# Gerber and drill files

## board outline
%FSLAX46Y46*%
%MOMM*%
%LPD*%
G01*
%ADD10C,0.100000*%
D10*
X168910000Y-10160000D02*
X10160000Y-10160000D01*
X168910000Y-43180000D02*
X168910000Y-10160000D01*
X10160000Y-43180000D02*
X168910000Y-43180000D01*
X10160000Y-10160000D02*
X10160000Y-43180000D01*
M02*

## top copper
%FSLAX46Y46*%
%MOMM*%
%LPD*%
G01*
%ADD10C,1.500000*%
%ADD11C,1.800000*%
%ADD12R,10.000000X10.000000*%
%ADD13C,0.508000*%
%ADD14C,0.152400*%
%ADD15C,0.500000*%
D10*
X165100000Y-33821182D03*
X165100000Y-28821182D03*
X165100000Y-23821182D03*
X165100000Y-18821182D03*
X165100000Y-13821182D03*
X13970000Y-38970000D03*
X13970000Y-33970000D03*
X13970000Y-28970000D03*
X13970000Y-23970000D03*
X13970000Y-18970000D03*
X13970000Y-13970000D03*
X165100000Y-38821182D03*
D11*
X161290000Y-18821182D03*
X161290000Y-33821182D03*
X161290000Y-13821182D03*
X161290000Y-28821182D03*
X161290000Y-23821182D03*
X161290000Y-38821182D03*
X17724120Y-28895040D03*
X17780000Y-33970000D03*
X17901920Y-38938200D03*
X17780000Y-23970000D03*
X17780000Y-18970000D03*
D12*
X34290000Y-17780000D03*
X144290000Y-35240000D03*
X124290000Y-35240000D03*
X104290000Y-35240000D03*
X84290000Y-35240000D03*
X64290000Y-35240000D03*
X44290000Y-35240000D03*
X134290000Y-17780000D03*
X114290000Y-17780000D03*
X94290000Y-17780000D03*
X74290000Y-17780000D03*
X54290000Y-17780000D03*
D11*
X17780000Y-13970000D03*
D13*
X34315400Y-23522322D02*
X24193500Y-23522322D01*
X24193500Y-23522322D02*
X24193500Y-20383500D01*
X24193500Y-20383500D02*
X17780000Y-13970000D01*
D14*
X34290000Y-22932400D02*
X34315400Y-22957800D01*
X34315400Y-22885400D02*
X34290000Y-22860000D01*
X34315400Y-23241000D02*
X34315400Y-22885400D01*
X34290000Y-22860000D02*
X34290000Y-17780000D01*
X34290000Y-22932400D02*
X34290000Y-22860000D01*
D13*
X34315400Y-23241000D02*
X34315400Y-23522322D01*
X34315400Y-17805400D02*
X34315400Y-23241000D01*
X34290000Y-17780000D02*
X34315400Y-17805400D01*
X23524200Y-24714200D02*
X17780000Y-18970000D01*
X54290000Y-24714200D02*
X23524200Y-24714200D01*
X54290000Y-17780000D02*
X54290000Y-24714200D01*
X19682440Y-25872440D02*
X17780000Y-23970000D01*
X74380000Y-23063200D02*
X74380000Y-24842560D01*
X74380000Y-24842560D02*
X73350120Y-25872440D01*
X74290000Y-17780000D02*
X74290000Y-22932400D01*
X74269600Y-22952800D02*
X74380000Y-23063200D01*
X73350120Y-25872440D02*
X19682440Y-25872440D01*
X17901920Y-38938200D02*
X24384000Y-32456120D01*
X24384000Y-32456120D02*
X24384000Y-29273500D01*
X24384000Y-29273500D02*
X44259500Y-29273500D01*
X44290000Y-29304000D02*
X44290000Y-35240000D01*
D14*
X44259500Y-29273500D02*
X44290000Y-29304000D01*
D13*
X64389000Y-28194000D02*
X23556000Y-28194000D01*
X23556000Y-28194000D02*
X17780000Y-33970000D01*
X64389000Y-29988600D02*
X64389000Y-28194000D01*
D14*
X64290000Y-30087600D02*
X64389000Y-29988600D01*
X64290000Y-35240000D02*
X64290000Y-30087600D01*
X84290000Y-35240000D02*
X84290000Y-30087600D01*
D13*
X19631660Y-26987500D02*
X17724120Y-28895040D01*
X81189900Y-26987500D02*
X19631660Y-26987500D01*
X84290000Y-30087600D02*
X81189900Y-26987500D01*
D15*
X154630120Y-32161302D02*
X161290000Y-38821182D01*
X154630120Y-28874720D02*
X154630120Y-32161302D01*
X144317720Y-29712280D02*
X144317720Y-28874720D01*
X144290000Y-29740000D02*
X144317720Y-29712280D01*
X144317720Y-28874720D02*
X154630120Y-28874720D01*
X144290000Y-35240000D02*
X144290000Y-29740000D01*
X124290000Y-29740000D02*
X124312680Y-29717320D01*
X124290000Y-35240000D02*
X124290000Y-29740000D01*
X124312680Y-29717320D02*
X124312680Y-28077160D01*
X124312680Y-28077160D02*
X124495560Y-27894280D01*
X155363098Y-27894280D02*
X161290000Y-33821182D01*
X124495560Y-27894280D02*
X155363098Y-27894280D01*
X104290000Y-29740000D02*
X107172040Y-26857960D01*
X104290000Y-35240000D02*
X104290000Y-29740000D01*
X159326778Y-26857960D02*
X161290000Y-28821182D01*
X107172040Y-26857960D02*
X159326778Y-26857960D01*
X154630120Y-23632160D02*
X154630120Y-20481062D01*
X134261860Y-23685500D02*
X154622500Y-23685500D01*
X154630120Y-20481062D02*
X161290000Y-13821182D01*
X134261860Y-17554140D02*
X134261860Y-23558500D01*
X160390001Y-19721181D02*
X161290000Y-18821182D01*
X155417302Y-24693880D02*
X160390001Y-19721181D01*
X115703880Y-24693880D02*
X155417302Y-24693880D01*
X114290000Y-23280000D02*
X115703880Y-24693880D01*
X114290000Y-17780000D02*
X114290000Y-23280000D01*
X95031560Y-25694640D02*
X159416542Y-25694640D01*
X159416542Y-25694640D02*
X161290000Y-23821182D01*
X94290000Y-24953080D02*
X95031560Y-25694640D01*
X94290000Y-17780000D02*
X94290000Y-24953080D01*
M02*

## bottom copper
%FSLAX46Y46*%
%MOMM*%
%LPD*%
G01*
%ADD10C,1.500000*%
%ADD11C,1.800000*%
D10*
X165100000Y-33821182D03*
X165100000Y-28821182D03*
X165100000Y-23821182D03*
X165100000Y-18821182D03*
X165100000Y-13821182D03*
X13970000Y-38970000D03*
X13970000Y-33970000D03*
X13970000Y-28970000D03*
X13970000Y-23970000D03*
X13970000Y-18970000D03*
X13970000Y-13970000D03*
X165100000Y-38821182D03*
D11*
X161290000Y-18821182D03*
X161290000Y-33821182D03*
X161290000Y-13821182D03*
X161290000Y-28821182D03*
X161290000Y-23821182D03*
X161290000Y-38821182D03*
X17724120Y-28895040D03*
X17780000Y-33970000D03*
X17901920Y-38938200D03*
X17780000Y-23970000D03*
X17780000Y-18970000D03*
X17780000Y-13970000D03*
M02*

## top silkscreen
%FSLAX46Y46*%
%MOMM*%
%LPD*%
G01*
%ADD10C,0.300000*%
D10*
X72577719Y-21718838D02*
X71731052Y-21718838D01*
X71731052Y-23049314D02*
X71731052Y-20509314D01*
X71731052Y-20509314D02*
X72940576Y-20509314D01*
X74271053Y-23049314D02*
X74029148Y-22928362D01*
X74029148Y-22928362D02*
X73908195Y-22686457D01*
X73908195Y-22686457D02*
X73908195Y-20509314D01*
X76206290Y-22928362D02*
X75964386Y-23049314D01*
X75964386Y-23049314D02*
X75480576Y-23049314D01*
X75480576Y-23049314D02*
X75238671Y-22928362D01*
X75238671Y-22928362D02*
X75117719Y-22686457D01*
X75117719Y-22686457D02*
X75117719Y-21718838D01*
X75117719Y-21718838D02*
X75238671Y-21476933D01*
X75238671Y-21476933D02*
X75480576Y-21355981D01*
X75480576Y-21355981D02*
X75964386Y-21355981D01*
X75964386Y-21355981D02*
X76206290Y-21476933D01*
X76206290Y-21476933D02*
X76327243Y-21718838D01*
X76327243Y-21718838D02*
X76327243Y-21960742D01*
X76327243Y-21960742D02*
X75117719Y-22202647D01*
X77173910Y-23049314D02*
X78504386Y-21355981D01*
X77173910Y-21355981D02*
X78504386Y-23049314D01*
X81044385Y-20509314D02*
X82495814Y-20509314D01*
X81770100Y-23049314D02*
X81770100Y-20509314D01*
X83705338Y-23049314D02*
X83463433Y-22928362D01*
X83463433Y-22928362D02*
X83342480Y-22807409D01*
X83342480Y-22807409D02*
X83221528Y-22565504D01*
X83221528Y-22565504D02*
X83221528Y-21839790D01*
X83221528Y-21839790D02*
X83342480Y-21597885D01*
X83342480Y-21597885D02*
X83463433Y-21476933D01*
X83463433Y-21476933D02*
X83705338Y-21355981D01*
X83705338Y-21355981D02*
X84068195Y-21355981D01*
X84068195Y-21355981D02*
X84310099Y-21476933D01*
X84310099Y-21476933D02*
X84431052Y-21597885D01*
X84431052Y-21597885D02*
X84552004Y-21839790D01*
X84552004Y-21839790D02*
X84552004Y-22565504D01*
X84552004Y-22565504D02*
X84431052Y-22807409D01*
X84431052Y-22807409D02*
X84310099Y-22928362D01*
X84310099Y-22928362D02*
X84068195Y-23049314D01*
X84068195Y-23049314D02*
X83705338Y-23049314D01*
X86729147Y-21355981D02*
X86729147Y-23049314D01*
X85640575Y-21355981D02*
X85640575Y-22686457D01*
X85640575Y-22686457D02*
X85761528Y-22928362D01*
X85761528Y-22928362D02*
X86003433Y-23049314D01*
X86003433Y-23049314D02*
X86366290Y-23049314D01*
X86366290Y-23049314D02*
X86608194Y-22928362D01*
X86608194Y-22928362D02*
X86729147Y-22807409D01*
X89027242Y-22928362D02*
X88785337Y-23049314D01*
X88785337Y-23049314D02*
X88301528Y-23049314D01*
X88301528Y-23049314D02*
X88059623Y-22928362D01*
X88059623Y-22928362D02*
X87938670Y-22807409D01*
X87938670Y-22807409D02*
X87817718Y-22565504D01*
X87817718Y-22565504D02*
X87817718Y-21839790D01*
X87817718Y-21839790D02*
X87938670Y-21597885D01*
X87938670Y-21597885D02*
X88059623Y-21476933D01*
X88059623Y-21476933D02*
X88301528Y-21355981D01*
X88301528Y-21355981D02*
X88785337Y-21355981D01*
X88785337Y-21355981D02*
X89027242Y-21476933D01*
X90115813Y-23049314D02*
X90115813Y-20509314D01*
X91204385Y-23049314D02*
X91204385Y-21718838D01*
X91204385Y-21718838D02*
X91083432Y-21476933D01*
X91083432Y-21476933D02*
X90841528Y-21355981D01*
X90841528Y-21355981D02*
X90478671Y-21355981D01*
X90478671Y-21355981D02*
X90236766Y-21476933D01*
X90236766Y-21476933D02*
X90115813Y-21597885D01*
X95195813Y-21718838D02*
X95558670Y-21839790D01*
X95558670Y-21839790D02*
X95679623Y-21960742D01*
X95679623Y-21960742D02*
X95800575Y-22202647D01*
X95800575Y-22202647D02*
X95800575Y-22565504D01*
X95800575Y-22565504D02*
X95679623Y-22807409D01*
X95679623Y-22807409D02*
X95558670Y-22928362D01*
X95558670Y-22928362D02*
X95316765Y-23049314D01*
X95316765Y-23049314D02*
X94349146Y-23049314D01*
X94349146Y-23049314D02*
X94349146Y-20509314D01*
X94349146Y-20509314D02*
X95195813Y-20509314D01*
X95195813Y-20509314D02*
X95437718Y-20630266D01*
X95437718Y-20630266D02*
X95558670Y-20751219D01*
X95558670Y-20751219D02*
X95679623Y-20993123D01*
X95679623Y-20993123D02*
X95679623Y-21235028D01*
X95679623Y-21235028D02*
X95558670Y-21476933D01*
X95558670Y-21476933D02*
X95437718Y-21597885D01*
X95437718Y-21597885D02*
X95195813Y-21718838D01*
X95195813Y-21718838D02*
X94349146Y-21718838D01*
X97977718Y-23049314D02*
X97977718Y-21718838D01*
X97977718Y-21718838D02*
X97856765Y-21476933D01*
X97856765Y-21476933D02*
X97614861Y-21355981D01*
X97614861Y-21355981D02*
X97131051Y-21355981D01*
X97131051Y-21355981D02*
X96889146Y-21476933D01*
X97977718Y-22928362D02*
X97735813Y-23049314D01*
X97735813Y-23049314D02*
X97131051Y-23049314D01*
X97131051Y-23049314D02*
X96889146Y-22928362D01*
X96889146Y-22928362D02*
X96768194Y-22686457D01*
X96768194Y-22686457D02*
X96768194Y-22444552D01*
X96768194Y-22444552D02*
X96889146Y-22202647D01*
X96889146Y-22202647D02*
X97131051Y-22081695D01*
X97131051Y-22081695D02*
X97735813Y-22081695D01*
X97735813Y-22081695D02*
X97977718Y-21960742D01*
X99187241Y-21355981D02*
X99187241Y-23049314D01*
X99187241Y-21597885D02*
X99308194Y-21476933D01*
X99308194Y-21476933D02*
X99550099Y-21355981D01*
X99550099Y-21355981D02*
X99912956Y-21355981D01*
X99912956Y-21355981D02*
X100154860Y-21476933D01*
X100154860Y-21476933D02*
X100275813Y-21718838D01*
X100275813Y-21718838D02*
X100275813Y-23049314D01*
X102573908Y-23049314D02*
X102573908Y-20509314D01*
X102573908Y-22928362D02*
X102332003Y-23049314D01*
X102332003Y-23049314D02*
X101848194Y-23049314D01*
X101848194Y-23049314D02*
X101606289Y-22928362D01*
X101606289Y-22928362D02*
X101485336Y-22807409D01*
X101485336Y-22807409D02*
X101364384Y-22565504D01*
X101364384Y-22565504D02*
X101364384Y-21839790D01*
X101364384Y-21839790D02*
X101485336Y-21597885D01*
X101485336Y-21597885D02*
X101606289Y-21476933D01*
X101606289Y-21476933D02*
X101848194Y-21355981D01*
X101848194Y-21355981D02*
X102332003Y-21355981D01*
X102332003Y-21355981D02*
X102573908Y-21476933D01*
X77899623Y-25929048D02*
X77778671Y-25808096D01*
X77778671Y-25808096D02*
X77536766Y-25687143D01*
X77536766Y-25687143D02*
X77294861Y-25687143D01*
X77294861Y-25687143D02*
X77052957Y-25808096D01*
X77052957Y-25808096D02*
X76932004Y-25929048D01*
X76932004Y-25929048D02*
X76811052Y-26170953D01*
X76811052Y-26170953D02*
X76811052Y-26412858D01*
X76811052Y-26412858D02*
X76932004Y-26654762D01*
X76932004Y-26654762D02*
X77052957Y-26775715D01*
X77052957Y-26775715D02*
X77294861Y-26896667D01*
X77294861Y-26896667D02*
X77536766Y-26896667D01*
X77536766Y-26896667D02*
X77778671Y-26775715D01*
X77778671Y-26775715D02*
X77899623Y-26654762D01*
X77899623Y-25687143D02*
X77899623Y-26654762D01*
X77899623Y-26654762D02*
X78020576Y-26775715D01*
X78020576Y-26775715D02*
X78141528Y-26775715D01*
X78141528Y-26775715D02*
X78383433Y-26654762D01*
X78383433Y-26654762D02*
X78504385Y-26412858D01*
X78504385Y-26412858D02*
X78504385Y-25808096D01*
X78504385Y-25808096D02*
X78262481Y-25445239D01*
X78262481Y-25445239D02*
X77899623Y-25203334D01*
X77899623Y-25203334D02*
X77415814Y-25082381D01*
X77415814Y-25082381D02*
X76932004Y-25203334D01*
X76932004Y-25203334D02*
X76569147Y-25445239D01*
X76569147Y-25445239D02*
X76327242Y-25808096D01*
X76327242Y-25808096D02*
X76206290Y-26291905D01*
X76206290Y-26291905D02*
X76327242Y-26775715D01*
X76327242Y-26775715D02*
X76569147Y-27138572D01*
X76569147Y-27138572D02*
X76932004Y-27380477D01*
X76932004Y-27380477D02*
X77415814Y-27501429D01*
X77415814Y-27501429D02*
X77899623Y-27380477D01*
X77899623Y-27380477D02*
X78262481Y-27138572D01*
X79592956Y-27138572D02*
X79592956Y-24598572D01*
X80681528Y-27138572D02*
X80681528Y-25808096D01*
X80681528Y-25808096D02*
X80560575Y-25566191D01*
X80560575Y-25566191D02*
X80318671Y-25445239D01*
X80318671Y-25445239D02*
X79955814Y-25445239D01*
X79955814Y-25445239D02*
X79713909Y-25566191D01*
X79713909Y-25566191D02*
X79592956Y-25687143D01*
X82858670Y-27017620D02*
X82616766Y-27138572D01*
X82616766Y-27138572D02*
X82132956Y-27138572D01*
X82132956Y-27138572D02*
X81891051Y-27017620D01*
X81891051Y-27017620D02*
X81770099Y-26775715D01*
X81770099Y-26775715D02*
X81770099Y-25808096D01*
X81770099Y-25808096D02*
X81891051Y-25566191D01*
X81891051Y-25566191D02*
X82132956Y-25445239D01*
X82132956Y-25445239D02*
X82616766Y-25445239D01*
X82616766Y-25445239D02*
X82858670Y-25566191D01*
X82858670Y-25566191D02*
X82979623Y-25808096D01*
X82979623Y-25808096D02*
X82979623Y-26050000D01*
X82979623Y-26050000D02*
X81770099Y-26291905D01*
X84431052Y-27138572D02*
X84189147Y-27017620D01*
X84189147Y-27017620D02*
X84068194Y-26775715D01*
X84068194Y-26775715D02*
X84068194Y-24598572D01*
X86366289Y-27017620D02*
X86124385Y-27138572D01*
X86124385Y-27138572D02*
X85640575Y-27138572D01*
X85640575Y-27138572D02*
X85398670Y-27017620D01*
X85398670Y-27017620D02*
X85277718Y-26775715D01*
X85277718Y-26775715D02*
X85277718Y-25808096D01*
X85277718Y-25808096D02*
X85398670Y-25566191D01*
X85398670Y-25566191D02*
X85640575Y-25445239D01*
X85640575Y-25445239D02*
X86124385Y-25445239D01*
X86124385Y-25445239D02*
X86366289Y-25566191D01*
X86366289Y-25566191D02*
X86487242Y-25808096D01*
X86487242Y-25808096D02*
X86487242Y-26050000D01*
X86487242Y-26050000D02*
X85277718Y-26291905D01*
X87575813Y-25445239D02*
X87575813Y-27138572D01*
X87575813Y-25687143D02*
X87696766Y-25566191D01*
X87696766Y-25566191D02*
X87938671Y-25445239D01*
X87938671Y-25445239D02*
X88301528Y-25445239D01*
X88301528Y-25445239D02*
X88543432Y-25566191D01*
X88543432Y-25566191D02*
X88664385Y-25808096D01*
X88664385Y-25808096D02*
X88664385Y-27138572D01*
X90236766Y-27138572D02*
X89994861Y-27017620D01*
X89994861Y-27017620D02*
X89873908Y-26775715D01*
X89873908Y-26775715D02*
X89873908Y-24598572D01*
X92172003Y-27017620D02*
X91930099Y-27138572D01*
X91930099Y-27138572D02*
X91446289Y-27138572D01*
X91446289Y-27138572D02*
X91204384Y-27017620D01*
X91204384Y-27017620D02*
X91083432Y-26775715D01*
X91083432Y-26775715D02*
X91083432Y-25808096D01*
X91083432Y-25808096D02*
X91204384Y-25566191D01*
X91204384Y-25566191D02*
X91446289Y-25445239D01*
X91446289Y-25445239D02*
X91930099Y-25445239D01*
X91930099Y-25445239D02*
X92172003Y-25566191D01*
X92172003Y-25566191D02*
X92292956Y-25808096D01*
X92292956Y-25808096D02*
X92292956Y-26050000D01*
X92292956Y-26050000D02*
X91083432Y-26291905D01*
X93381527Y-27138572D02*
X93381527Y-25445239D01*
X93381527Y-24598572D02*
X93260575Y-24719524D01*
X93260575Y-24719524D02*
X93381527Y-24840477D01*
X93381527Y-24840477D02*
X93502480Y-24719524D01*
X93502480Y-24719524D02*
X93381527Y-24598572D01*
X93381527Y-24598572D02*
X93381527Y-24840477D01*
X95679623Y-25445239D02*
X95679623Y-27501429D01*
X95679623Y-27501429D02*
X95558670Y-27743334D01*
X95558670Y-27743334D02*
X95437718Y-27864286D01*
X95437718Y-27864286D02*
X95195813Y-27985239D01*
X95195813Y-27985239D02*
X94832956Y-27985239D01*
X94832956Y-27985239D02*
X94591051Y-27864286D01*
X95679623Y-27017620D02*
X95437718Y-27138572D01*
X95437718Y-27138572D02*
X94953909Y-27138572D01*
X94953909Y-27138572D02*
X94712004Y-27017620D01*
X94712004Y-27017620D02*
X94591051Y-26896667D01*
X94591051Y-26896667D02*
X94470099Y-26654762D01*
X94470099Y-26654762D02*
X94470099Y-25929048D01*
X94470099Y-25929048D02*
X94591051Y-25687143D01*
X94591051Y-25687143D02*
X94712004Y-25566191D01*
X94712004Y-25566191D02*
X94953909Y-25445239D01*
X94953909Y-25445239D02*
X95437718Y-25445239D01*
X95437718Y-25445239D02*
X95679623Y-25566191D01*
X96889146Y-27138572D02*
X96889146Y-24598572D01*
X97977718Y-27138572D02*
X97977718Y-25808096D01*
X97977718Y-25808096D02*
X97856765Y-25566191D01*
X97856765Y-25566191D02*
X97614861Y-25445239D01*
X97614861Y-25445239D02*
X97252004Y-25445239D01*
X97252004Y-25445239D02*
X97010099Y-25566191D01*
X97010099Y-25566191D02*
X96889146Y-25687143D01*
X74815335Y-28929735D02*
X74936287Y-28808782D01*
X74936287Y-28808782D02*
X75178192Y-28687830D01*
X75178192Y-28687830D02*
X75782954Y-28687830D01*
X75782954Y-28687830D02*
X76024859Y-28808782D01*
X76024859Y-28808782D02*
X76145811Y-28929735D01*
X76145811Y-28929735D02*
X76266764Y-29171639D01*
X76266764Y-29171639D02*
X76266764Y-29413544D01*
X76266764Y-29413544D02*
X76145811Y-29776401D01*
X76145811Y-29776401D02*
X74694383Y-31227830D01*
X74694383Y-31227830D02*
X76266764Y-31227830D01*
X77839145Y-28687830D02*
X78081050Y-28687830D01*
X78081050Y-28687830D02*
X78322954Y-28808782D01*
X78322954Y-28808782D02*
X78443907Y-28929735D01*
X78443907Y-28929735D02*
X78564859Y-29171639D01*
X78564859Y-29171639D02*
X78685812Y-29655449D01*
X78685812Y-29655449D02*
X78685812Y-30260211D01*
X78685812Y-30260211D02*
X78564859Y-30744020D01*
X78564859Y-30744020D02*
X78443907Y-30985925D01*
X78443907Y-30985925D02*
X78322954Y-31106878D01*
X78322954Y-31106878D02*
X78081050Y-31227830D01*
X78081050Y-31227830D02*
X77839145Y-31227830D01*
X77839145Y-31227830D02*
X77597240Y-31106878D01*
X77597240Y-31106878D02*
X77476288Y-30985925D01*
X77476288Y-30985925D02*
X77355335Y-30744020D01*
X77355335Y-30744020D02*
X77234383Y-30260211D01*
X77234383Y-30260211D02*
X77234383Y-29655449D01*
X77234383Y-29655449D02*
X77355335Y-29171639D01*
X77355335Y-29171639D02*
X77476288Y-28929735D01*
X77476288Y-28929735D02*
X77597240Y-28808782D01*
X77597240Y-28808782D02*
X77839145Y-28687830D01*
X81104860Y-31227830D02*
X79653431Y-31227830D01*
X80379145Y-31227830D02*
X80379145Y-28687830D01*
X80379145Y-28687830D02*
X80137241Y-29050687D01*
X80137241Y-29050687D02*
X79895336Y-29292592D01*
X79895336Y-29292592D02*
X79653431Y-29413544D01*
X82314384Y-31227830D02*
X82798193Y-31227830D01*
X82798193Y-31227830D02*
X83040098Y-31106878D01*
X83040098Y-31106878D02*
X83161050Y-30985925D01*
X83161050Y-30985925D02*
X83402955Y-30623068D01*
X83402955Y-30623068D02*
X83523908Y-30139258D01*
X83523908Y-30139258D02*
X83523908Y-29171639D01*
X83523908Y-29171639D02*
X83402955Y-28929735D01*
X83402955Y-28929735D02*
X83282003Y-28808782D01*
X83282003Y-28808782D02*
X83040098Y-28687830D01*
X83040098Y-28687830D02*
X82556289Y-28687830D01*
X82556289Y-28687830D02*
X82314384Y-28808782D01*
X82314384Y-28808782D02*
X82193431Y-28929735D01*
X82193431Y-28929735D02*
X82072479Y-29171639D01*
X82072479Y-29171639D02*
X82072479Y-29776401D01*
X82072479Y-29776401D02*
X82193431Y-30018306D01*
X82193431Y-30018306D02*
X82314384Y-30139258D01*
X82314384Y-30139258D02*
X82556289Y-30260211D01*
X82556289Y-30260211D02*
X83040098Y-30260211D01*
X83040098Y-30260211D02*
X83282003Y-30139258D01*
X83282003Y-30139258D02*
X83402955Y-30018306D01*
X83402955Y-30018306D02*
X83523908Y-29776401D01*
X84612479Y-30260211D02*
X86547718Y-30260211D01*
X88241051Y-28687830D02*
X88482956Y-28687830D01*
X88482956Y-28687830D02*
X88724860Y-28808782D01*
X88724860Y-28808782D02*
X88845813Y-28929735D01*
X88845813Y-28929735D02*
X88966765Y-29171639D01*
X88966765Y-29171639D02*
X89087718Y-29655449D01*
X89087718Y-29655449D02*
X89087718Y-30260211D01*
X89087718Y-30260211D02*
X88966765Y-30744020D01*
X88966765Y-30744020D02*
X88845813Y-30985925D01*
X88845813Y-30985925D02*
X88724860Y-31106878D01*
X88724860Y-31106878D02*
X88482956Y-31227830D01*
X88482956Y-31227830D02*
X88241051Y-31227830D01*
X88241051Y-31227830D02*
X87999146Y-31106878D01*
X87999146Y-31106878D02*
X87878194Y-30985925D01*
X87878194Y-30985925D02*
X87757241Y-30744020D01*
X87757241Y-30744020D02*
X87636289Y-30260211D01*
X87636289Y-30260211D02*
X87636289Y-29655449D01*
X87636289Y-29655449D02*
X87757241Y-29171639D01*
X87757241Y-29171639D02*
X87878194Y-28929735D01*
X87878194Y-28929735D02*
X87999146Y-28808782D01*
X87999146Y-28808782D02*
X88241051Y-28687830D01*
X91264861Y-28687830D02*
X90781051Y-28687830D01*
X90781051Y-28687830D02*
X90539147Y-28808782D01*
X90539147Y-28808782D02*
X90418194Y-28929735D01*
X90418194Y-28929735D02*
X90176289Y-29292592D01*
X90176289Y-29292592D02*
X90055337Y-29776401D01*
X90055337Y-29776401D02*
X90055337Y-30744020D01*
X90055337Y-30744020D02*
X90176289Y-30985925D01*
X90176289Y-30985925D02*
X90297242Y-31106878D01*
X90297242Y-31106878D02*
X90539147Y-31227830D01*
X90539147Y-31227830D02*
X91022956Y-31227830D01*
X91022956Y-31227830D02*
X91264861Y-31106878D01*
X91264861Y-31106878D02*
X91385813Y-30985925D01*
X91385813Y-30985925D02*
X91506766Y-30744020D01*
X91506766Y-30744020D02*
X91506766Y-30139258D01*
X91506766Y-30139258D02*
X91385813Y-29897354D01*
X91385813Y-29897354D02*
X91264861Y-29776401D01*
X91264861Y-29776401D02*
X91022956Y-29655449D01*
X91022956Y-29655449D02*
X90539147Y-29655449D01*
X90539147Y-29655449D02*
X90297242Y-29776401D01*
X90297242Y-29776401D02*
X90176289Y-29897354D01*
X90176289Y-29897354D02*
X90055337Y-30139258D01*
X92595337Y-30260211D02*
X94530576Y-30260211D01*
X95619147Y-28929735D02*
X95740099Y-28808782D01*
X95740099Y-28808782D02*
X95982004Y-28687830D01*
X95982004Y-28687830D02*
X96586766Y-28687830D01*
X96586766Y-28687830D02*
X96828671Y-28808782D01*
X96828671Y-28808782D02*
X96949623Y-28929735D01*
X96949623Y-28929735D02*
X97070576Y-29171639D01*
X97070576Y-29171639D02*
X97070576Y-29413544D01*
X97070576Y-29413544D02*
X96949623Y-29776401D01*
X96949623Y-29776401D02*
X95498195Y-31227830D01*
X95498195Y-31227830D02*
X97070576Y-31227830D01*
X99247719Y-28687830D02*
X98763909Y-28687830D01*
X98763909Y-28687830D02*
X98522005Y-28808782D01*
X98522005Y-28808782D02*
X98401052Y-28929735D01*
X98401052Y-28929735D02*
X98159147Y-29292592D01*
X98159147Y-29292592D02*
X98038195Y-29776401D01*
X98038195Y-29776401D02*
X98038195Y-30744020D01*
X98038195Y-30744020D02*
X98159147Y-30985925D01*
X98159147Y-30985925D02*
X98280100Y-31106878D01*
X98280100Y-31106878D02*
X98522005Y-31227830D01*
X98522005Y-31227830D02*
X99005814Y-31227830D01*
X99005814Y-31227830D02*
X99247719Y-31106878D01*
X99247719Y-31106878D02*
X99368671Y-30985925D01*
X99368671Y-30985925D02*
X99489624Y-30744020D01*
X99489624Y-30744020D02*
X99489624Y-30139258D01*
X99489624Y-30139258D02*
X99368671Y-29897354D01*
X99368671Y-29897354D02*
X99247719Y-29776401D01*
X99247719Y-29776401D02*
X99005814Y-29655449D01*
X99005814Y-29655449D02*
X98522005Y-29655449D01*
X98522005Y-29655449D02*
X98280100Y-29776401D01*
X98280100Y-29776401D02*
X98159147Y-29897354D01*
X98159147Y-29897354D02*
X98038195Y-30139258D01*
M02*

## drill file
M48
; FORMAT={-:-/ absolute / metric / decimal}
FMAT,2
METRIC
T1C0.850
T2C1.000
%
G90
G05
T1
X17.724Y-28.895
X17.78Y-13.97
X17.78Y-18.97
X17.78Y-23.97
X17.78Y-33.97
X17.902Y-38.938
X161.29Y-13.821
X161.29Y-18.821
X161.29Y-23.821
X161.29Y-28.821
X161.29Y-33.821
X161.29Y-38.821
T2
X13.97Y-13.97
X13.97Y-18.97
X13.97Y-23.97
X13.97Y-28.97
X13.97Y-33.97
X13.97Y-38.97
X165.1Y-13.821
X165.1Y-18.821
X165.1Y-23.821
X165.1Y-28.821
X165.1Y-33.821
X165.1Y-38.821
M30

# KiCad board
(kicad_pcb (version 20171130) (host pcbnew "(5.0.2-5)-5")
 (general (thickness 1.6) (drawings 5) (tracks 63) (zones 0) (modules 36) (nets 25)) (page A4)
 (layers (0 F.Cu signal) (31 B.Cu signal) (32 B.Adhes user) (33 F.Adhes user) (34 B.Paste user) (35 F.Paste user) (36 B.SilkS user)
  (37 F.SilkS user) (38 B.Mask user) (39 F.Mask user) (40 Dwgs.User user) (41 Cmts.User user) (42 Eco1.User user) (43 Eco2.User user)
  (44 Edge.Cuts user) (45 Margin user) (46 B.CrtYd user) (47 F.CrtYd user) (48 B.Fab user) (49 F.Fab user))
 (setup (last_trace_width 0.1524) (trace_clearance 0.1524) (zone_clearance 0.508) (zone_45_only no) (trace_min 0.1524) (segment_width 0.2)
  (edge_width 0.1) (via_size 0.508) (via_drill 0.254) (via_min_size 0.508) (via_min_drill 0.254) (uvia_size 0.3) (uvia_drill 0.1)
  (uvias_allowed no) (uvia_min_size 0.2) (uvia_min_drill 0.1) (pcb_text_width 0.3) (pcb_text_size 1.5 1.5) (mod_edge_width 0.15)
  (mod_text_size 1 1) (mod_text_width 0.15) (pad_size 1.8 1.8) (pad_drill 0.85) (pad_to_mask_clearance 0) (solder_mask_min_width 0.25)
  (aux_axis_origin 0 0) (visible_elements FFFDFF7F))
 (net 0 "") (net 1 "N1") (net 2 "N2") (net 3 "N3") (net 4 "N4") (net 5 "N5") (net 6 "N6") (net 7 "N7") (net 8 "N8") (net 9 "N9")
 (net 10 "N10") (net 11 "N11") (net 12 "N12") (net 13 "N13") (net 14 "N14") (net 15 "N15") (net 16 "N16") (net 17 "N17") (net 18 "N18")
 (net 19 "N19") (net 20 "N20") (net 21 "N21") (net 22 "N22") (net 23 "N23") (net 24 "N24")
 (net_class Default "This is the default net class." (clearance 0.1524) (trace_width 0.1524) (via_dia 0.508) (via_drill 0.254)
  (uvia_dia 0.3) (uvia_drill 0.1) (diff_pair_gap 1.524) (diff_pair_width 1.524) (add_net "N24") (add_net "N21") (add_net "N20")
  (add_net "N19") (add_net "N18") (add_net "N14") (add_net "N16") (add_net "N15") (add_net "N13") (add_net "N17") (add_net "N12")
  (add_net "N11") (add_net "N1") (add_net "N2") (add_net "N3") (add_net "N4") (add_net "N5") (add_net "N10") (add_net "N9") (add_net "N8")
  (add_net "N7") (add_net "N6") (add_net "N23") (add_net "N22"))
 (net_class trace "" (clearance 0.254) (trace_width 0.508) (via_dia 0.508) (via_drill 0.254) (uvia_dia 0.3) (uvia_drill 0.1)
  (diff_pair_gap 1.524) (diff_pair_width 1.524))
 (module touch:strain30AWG (layer B.Cu) (at 165.1 33.821182)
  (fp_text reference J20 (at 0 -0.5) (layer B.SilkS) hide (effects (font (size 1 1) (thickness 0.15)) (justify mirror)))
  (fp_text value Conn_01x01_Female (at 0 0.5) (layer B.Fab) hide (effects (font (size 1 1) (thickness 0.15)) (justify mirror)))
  (pad 1 thru_hole circle (at 0 0) (size 1.5 1.5) (drill 1) (layers *.Cu) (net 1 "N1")))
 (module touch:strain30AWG (layer B.Cu) (at 165.1 28.821182)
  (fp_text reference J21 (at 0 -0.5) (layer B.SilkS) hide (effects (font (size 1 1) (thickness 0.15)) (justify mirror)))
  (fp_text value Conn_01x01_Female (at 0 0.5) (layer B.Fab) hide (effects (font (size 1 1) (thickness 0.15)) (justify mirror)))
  (pad 1 thru_hole circle (at 0 0) (size 1.5 1.5) (drill 1) (layers *.Cu) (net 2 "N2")))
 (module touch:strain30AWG (layer B.Cu) (at 165.1 23.821182)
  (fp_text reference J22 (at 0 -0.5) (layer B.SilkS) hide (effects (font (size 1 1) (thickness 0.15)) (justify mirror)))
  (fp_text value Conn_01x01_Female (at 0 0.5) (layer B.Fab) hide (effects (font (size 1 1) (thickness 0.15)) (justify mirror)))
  (pad 1 thru_hole circle (at 0 0) (size 1.5 1.5) (drill 1) (layers *.Cu) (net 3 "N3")))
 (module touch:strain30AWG (layer B.Cu) (at 165.1 18.821182)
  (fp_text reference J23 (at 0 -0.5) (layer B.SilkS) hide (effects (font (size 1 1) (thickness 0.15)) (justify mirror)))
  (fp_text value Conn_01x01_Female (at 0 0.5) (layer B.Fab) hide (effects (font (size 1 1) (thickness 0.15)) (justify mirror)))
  (pad 1 thru_hole circle (at 0 0) (size 1.5 1.5) (drill 1) (layers *.Cu) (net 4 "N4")))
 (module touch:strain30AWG (layer B.Cu) (at 165.1 13.821182)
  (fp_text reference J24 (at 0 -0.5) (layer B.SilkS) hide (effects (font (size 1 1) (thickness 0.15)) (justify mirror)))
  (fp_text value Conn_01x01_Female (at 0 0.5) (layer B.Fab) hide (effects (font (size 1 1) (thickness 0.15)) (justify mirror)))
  (pad 1 thru_hole circle (at 0 0) (size 1.5 1.5) (drill 1) (layers *.Cu) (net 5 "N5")))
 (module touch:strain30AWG (layer F.Cu) (at 13.97 38.97)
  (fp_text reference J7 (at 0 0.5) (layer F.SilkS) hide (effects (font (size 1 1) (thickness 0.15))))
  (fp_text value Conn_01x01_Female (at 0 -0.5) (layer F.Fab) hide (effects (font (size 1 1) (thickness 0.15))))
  (pad 1 thru_hole circle (at 0 0) (size 1.5 1.5) (drill 1) (layers *.Cu) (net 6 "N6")))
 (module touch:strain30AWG (layer F.Cu) (at 13.97 33.97)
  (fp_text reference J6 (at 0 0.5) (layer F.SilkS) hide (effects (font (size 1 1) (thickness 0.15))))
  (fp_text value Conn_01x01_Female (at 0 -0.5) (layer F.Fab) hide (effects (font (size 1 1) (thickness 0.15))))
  (pad 1 thru_hole circle (at 0 0) (size 1.5 1.5) (drill 1) (layers *.Cu) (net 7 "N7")))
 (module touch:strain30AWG (layer F.Cu) (at 13.97 28.97)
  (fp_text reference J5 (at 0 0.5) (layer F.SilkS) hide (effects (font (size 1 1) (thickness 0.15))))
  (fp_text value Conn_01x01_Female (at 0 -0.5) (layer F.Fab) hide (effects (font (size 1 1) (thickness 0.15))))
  (pad 1 thru_hole circle (at 0 0) (size 1.5 1.5) (drill 1) (layers *.Cu) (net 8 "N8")))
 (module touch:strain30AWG (layer F.Cu) (at 13.97 23.97)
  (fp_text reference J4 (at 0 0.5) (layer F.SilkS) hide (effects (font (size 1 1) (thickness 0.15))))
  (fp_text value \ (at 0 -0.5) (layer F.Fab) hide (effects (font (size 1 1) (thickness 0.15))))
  (pad 1 thru_hole circle (at 0 0) (size 1.5 1.5) (drill 1) (layers *.Cu) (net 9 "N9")))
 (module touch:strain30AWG (layer F.Cu) (at 13.97 18.97)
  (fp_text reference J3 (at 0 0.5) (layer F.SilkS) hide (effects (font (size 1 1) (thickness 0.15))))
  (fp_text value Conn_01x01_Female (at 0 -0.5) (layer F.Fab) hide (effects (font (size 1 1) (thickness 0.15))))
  (pad 1 thru_hole circle (at 0 0) (size 1.5 1.5) (drill 1) (layers *.Cu) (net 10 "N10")))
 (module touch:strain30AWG (layer F.Cu) (at 13.97 13.97)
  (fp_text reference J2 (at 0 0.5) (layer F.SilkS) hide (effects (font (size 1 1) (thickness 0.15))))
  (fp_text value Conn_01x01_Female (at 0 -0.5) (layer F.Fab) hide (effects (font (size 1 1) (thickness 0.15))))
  (pad 1 thru_hole circle (at 0 0) (size 1.5 1.5) (drill 1) (layers *.Cu) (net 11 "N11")))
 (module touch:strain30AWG (layer B.Cu) (at 165.1 38.821182)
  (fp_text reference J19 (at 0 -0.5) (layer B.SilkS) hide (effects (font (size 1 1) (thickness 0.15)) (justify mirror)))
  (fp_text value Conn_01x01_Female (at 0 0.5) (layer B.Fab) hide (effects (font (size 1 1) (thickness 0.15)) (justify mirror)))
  (pad 1 thru_hole circle (at 0 0) (size 1.5 1.5) (drill 1) (layers *.Cu) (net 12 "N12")))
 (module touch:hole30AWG (layer B.Cu) (at 161.29 18.821182)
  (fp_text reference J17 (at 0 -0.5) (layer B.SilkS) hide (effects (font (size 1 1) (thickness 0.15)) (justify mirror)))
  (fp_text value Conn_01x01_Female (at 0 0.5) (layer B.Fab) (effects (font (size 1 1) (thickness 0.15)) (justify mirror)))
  (pad 1 thru_hole circle (at 0 0) (size 1.8 1.8) (drill 0.85) (layers *.Cu *.Mask) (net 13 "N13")))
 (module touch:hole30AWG (layer B.Cu) (at 161.29 33.821182)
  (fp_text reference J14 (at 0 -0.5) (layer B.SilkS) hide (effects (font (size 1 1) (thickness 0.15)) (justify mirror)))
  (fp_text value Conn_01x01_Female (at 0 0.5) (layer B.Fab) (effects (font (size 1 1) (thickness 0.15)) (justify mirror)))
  (pad 1 thru_hole circle (at 0 0) (size 1.8 1.8) (drill 0.85) (layers *.Cu *.Mask) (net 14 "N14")))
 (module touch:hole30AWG (layer B.Cu) (at 161.29 13.821182)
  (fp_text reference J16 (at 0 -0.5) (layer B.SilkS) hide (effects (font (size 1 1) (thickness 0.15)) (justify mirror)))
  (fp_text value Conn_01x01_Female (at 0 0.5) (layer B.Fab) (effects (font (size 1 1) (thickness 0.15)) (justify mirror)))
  (pad 1 thru_hole circle (at 0 0) (size 1.8 1.8) (drill 0.85) (layers *.Cu *.Mask) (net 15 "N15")))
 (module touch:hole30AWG (layer B.Cu) (at 161.29 28.821182)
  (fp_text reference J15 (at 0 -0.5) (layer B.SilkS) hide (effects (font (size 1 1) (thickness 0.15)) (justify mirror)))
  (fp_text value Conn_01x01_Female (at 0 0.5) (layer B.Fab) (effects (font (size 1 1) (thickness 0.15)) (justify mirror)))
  (pad 1 thru_hole circle (at 0 0) (size 1.8 1.8) (drill 0.85) (layers *.Cu *.Mask) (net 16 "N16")))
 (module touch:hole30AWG (layer B.Cu) (at 161.29 23.821182)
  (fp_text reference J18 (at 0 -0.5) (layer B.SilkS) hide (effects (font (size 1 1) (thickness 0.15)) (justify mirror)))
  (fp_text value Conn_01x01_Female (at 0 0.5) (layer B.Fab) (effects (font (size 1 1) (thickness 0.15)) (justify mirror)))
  (pad 1 thru_hole circle (at 0 0) (size 1.8 1.8) (drill 0.85) (layers *.Cu *.Mask) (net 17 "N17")))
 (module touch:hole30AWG (layer B.Cu) (at 161.29 38.821182)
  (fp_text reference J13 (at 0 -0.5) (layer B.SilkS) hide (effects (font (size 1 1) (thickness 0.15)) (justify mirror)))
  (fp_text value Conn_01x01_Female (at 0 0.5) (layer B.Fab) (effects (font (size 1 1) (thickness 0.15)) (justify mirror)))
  (pad 1 thru_hole circle (at 0 0) (size 1.8 1.8) (drill 0.85) (layers *.Cu *.Mask) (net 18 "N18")))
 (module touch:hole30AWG (layer F.Cu) (at 17.72412 28.89504)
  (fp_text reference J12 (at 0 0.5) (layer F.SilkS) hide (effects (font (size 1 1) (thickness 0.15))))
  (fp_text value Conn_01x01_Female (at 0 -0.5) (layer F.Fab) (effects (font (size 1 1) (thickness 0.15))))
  (pad 1 thru_hole circle (at 0 0) (size 1.8 1.8) (drill 0.85) (layers *.Cu *.Mask) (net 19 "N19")))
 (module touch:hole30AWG (layer F.Cu) (at 17.78 33.97)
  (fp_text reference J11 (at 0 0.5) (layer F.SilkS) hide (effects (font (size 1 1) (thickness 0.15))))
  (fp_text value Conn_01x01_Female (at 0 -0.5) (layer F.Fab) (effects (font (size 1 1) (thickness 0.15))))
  (pad 1 thru_hole circle (at 0 0) (size 1.8 1.8) (drill 0.85) (layers *.Cu *.Mask) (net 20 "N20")))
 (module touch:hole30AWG (layer F.Cu) (at 17.90192 38.9382)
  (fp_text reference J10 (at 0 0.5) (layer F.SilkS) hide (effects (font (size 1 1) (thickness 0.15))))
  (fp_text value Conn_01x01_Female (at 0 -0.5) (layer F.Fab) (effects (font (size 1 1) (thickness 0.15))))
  (pad 1 thru_hole circle (at 0 0) (size 1.8 1.8) (drill 0.85) (layers *.Cu *.Mask) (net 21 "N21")))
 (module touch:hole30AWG (layer F.Cu) (at 17.78 23.97)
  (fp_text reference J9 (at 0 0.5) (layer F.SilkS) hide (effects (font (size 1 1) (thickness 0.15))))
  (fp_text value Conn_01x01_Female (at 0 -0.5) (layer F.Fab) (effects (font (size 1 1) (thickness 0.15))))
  (pad 1 thru_hole circle (at 0 0) (size 1.8 1.8) (drill 0.85) (layers *.Cu *.Mask) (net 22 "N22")))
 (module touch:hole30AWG (layer F.Cu) (at 17.78 18.97)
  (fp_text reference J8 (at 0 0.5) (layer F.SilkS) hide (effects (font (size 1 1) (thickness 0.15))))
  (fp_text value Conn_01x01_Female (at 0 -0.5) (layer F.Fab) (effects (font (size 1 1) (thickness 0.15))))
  (pad 1 thru_hole circle (at 0 0) (size 1.8 1.8) (drill 0.85) (layers *.Cu *.Mask) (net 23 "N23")))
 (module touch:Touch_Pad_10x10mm (layer F.Cu) (at 34.29 17.78)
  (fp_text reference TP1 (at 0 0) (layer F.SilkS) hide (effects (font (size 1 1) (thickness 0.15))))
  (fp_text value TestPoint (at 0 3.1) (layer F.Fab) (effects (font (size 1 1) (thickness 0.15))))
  (pad 1 smd rect (at 0 0) (size 10 10) (layers F.Cu F.Mask) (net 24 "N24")))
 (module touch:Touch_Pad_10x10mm (layer F.Cu) (at 144.29 35.24)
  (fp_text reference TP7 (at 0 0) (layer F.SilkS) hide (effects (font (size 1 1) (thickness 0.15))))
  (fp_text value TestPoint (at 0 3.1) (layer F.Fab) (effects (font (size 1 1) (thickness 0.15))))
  (pad 1 smd rect (at 0 0) (size 10 10) (layers F.Cu F.Mask) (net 18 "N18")))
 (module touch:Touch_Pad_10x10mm (layer F.Cu) (at 124.29 35.24)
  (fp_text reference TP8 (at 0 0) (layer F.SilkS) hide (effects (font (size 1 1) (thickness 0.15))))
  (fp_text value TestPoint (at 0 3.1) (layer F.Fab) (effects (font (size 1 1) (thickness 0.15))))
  (pad 1 smd rect (at 0 0) (size 10 10) (layers F.Cu F.Mask) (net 14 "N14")))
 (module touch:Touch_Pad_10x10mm (layer F.Cu) (at 104.29 35.24)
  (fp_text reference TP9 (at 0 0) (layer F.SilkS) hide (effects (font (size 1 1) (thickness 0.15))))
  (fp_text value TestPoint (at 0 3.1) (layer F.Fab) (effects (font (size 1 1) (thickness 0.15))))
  (pad 1 smd rect (at 0 0) (size 10 10) (layers F.Cu F.Mask) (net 16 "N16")))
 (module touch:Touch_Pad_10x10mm (layer F.Cu) (at 84.29 35.24)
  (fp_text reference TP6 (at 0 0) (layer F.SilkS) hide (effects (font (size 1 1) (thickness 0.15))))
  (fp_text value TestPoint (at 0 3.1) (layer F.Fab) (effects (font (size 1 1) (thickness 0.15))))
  (pad 1 smd rect (at 0 0) (size 10 10) (layers F.Cu F.Mask) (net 19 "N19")))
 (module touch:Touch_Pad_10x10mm (layer F.Cu) (at 64.29 35.24)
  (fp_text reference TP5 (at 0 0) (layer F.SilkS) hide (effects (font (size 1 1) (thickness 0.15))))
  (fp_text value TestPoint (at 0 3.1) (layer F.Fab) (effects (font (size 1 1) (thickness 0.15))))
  (pad 1 smd rect (at 0 0) (size 10 10) (layers F.Cu F.Mask) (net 20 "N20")))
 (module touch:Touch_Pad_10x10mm (layer F.Cu) (at 44.29 35.24)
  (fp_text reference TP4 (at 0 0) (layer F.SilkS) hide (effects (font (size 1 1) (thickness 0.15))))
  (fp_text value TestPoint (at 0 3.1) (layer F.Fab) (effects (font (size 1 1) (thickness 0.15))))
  (pad 1 smd rect (at 0 0) (size 10 10) (layers F.Cu F.Mask) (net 21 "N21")))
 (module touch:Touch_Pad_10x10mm (layer F.Cu) (at 134.29 17.78)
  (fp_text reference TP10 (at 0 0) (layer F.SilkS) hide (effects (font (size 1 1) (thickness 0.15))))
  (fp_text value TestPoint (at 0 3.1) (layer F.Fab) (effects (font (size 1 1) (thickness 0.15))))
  (pad 1 smd rect (at 0 0) (size 10 10) (layers F.Cu F.Mask) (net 15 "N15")))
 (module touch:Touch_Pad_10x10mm (layer F.Cu) (at 114.29 17.78)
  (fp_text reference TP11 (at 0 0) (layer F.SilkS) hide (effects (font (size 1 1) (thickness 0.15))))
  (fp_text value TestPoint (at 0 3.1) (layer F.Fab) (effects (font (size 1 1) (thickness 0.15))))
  (pad 1 smd rect (at 0 0) (size 10 10) (layers F.Cu F.Mask) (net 13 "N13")))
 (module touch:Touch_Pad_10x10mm (layer F.Cu) (at 94.29 17.78)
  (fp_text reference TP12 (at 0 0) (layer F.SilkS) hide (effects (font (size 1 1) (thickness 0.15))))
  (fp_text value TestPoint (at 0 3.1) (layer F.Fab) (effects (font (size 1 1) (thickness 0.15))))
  (pad 1 smd rect (at 0 0) (size 10 10) (layers F.Cu F.Mask) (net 17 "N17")))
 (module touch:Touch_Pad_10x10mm (layer F.Cu) (at 74.29 17.78)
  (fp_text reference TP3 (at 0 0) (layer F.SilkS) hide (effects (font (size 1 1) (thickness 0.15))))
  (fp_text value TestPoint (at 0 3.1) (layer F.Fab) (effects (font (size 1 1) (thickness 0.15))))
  (pad 1 smd rect (at 0 0) (size 10 10) (layers F.Cu F.Mask) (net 22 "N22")))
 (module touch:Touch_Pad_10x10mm (layer F.Cu) (at 54.29 17.78)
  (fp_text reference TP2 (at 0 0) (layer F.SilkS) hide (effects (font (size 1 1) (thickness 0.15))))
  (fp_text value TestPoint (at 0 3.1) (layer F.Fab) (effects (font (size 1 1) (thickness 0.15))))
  (pad 1 smd rect (at 0 0) (size 10 10) (layers F.Cu F.Mask) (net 23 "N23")))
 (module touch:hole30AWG (layer F.Cu) (at 17.78 13.97)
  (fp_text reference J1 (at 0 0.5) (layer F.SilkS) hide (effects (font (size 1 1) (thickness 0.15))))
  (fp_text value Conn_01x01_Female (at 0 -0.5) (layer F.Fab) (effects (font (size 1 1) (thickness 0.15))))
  (pad 1 thru_hole circle (at 0 0) (size 1.8 1.8) (drill 0.85) (layers *.Cu *.Mask) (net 24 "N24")))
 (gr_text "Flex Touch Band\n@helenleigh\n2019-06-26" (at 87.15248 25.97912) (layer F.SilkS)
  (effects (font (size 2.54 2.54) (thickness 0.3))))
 (gr_line (start 168.91 10.16) (end 10.16 10.16) (layer Edge.Cuts) (width 0.1))
 (gr_line (start 168.91 43.18) (end 168.91 10.16) (layer Edge.Cuts) (width 0.1))
 (gr_line (start 10.16 43.18) (end 168.91 43.18) (layer Edge.Cuts) (width 0.1))
 (gr_line (start 10.16 10.16) (end 10.16 43.18) (layer Edge.Cuts) (width 0.1))
 (segment (start 34.3154 23.522322) (end 24.1935 23.522322) (width 0.508) (layer F.Cu) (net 24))
 (segment (start 24.1935 23.522322) (end 24.1935 20.3835) (width 0.508) (layer F.Cu) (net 24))
 (segment (start 24.1935 20.3835) (end 17.78 13.97) (width 0.508) (layer F.Cu) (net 24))
 (segment (start 34.29 22.9324) (end 34.3154 22.9578) (width 0.1524) (layer F.Cu) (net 24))
 (segment (start 34.3154 22.8854) (end 34.29 22.86) (width 0.1524) (layer F.Cu) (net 24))
 (segment (start 34.3154 23.241) (end 34.3154 22.8854) (width 0.1524) (layer F.Cu) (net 24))
 (segment (start 34.29 22.86) (end 34.29 17.78) (width 0.1524) (layer F.Cu) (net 24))
 (segment (start 34.29 22.9324) (end 34.29 22.86) (width 0.1524) (layer F.Cu) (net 24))
 (segment (start 34.3154 23.241) (end 34.3154 23.522322) (width 0.508) (layer F.Cu) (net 24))
 (segment (start 34.3154 17.8054) (end 34.3154 23.241) (width 0.508) (layer F.Cu) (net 24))
 (segment (start 34.29 17.78) (end 34.3154 17.8054) (width 0.508) (layer F.Cu) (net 24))
 (segment (start 23.5242 24.7142) (end 17.78 18.97) (width 0.508) (layer F.Cu) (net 23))
 (segment (start 54.29 24.7142) (end 23.5242 24.7142) (width 0.508) (layer F.Cu) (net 23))
 (segment (start 54.29 17.78) (end 54.29 24.7142) (width 0.508) (layer F.Cu) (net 23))
 (segment (start 19.68244 25.87244) (end 17.78 23.97) (width 0.508) (layer F.Cu) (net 22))
 (segment (start 74.38 23.0632) (end 74.38 24.84256) (width 0.508) (layer F.Cu) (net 22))
 (segment (start 74.38 24.84256) (end 73.35012 25.87244) (width 0.508) (layer F.Cu) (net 22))
 (segment (start 74.29 17.78) (end 74.29 22.9324) (width 0.508) (layer F.Cu) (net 22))
 (segment (start 74.2696 22.9528) (end 74.38 23.0632) (width 0.508) (layer F.Cu) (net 22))
 (segment (start 73.35012 25.87244) (end 19.68244 25.87244) (width 0.508) (layer F.Cu) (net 22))
 (segment (start 17.90192 38.9382) (end 24.384 32.45612) (width 0.508) (layer F.Cu) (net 21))
 (segment (start 24.384 32.45612) (end 24.384 29.2735) (width 0.508) (layer F.Cu) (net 21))
 (segment (start 24.384 29.2735) (end 44.2595 29.2735) (width 0.508) (layer F.Cu) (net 21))
 (segment (start 44.29 29.304) (end 44.29 35.24) (width 0.508) (layer F.Cu) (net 21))
 (segment (start 44.2595 29.2735) (end 44.29 29.304) (width 0.1524) (layer F.Cu) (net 21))
 (segment (start 64.389 28.194) (end 23.556 28.194) (width 0.508) (layer F.Cu) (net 20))
 (segment (start 23.556 28.194) (end 17.78 33.97) (width 0.508) (layer F.Cu) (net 20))
 (segment (start 64.389 29.9886) (end 64.389 28.194) (width 0.508) (layer F.Cu) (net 20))
 (segment (start 64.29 30.0876) (end 64.389 29.9886) (width 0.1524) (layer F.Cu) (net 20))
 (segment (start 64.29 35.24) (end 64.29 30.0876) (width 0.1524) (layer F.Cu) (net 20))
 (segment (start 84.29 35.24) (end 84.29 30.0876) (width 0.1524) (layer F.Cu) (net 19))
 (segment (start 19.63166 26.9875) (end 17.72412 28.89504) (width 0.508) (layer F.Cu) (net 19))
 (segment (start 81.1899 26.9875) (end 19.63166 26.9875) (width 0.508) (layer F.Cu) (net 19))
 (segment (start 84.29 30.0876) (end 81.1899 26.9875) (width 0.508) (layer F.Cu) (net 19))
 (segment (start 154.63012 32.161302) (end 161.29 38.821182) (width 0.5) (layer F.Cu) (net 18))
 (segment (start 154.63012 28.87472) (end 154.63012 32.161302) (width 0.5) (layer F.Cu) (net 18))
 (segment (start 144.31772 29.71228) (end 144.31772 28.87472) (width 0.5) (layer F.Cu) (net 18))
 (segment (start 144.29 29.74) (end 144.31772 29.71228) (width 0.5) (layer F.Cu) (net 18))
 (segment (start 144.31772 28.87472) (end 154.63012 28.87472) (width 0.5) (layer F.Cu) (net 18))
 (segment (start 144.29 35.24) (end 144.29 29.74) (width 0.5) (layer F.Cu) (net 18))
 (segment (start 124.29 29.74) (end 124.31268 29.71732) (width 0.5) (layer F.Cu) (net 14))
 (segment (start 124.29 35.24) (end 124.29 29.74) (width 0.5) (layer F.Cu) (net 14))
 (segment (start 124.31268 29.71732) (end 124.31268 28.07716) (width 0.5) (layer F.Cu) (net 14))
 (segment (start 124.31268 28.07716) (end 124.49556 27.89428) (width 0.5) (layer F.Cu) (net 14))
 (segment (start 155.363098 27.89428) (end 161.29 33.821182) (width 0.5) (layer F.Cu) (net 14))
 (segment (start 124.49556 27.89428) (end 155.363098 27.89428) (width 0.5) (layer F.Cu) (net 14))
 (segment (start 104.29 29.74) (end 107.17204 26.85796) (width 0.5) (layer F.Cu) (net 16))
 (segment (start 104.29 35.24) (end 104.29 29.74) (width 0.5) (layer F.Cu) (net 16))
 (segment (start 159.326778 26.85796) (end 161.29 28.821182) (width 0.5) (layer F.Cu) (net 16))
 (segment (start 107.17204 26.85796) (end 159.326778 26.85796) (width 0.5) (layer F.Cu) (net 16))
 (segment (start 154.63012 23.63216) (end 154.63012 20.481062) (width 0.5) (layer F.Cu) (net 15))
 (segment (start 134.26186 23.6855) (end 154.6225 23.6855) (width 0.5) (layer F.Cu) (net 15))
 (segment (start 154.63012 20.481062) (end 161.29 13.821182) (width 0.5) (layer F.Cu) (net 15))
 (segment (start 134.26186 17.55414) (end 134.26186 23.5585) (width 0.5) (layer F.Cu) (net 15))
 (segment (start 160.390001 19.721181) (end 161.29 18.821182) (width 0.5) (layer F.Cu) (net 13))
 (segment (start 155.417302 24.69388) (end 160.390001 19.721181) (width 0.5) (layer F.Cu) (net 13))
 (segment (start 115.70388 24.69388) (end 155.417302 24.69388) (width 0.5) (layer F.Cu) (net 13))
 (segment (start 114.29 23.28) (end 115.70388 24.69388) (width 0.5) (layer F.Cu) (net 13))
 (segment (start 114.29 17.78) (end 114.29 23.28) (width 0.5) (layer F.Cu) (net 13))
 (segment (start 95.03156 25.69464) (end 159.416542 25.69464) (width 0.5) (layer F.Cu) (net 17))
 (segment (start 159.416542 25.69464) (end 161.29 23.821182) (width 0.5) (layer F.Cu) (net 17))
 (segment (start 94.29 24.95308) (end 95.03156 25.69464) (width 0.5) (layer F.Cu) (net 17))
 (segment (start 94.29 17.78) (end 94.29 24.95308) (width 0.5) (layer F.Cu) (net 17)))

